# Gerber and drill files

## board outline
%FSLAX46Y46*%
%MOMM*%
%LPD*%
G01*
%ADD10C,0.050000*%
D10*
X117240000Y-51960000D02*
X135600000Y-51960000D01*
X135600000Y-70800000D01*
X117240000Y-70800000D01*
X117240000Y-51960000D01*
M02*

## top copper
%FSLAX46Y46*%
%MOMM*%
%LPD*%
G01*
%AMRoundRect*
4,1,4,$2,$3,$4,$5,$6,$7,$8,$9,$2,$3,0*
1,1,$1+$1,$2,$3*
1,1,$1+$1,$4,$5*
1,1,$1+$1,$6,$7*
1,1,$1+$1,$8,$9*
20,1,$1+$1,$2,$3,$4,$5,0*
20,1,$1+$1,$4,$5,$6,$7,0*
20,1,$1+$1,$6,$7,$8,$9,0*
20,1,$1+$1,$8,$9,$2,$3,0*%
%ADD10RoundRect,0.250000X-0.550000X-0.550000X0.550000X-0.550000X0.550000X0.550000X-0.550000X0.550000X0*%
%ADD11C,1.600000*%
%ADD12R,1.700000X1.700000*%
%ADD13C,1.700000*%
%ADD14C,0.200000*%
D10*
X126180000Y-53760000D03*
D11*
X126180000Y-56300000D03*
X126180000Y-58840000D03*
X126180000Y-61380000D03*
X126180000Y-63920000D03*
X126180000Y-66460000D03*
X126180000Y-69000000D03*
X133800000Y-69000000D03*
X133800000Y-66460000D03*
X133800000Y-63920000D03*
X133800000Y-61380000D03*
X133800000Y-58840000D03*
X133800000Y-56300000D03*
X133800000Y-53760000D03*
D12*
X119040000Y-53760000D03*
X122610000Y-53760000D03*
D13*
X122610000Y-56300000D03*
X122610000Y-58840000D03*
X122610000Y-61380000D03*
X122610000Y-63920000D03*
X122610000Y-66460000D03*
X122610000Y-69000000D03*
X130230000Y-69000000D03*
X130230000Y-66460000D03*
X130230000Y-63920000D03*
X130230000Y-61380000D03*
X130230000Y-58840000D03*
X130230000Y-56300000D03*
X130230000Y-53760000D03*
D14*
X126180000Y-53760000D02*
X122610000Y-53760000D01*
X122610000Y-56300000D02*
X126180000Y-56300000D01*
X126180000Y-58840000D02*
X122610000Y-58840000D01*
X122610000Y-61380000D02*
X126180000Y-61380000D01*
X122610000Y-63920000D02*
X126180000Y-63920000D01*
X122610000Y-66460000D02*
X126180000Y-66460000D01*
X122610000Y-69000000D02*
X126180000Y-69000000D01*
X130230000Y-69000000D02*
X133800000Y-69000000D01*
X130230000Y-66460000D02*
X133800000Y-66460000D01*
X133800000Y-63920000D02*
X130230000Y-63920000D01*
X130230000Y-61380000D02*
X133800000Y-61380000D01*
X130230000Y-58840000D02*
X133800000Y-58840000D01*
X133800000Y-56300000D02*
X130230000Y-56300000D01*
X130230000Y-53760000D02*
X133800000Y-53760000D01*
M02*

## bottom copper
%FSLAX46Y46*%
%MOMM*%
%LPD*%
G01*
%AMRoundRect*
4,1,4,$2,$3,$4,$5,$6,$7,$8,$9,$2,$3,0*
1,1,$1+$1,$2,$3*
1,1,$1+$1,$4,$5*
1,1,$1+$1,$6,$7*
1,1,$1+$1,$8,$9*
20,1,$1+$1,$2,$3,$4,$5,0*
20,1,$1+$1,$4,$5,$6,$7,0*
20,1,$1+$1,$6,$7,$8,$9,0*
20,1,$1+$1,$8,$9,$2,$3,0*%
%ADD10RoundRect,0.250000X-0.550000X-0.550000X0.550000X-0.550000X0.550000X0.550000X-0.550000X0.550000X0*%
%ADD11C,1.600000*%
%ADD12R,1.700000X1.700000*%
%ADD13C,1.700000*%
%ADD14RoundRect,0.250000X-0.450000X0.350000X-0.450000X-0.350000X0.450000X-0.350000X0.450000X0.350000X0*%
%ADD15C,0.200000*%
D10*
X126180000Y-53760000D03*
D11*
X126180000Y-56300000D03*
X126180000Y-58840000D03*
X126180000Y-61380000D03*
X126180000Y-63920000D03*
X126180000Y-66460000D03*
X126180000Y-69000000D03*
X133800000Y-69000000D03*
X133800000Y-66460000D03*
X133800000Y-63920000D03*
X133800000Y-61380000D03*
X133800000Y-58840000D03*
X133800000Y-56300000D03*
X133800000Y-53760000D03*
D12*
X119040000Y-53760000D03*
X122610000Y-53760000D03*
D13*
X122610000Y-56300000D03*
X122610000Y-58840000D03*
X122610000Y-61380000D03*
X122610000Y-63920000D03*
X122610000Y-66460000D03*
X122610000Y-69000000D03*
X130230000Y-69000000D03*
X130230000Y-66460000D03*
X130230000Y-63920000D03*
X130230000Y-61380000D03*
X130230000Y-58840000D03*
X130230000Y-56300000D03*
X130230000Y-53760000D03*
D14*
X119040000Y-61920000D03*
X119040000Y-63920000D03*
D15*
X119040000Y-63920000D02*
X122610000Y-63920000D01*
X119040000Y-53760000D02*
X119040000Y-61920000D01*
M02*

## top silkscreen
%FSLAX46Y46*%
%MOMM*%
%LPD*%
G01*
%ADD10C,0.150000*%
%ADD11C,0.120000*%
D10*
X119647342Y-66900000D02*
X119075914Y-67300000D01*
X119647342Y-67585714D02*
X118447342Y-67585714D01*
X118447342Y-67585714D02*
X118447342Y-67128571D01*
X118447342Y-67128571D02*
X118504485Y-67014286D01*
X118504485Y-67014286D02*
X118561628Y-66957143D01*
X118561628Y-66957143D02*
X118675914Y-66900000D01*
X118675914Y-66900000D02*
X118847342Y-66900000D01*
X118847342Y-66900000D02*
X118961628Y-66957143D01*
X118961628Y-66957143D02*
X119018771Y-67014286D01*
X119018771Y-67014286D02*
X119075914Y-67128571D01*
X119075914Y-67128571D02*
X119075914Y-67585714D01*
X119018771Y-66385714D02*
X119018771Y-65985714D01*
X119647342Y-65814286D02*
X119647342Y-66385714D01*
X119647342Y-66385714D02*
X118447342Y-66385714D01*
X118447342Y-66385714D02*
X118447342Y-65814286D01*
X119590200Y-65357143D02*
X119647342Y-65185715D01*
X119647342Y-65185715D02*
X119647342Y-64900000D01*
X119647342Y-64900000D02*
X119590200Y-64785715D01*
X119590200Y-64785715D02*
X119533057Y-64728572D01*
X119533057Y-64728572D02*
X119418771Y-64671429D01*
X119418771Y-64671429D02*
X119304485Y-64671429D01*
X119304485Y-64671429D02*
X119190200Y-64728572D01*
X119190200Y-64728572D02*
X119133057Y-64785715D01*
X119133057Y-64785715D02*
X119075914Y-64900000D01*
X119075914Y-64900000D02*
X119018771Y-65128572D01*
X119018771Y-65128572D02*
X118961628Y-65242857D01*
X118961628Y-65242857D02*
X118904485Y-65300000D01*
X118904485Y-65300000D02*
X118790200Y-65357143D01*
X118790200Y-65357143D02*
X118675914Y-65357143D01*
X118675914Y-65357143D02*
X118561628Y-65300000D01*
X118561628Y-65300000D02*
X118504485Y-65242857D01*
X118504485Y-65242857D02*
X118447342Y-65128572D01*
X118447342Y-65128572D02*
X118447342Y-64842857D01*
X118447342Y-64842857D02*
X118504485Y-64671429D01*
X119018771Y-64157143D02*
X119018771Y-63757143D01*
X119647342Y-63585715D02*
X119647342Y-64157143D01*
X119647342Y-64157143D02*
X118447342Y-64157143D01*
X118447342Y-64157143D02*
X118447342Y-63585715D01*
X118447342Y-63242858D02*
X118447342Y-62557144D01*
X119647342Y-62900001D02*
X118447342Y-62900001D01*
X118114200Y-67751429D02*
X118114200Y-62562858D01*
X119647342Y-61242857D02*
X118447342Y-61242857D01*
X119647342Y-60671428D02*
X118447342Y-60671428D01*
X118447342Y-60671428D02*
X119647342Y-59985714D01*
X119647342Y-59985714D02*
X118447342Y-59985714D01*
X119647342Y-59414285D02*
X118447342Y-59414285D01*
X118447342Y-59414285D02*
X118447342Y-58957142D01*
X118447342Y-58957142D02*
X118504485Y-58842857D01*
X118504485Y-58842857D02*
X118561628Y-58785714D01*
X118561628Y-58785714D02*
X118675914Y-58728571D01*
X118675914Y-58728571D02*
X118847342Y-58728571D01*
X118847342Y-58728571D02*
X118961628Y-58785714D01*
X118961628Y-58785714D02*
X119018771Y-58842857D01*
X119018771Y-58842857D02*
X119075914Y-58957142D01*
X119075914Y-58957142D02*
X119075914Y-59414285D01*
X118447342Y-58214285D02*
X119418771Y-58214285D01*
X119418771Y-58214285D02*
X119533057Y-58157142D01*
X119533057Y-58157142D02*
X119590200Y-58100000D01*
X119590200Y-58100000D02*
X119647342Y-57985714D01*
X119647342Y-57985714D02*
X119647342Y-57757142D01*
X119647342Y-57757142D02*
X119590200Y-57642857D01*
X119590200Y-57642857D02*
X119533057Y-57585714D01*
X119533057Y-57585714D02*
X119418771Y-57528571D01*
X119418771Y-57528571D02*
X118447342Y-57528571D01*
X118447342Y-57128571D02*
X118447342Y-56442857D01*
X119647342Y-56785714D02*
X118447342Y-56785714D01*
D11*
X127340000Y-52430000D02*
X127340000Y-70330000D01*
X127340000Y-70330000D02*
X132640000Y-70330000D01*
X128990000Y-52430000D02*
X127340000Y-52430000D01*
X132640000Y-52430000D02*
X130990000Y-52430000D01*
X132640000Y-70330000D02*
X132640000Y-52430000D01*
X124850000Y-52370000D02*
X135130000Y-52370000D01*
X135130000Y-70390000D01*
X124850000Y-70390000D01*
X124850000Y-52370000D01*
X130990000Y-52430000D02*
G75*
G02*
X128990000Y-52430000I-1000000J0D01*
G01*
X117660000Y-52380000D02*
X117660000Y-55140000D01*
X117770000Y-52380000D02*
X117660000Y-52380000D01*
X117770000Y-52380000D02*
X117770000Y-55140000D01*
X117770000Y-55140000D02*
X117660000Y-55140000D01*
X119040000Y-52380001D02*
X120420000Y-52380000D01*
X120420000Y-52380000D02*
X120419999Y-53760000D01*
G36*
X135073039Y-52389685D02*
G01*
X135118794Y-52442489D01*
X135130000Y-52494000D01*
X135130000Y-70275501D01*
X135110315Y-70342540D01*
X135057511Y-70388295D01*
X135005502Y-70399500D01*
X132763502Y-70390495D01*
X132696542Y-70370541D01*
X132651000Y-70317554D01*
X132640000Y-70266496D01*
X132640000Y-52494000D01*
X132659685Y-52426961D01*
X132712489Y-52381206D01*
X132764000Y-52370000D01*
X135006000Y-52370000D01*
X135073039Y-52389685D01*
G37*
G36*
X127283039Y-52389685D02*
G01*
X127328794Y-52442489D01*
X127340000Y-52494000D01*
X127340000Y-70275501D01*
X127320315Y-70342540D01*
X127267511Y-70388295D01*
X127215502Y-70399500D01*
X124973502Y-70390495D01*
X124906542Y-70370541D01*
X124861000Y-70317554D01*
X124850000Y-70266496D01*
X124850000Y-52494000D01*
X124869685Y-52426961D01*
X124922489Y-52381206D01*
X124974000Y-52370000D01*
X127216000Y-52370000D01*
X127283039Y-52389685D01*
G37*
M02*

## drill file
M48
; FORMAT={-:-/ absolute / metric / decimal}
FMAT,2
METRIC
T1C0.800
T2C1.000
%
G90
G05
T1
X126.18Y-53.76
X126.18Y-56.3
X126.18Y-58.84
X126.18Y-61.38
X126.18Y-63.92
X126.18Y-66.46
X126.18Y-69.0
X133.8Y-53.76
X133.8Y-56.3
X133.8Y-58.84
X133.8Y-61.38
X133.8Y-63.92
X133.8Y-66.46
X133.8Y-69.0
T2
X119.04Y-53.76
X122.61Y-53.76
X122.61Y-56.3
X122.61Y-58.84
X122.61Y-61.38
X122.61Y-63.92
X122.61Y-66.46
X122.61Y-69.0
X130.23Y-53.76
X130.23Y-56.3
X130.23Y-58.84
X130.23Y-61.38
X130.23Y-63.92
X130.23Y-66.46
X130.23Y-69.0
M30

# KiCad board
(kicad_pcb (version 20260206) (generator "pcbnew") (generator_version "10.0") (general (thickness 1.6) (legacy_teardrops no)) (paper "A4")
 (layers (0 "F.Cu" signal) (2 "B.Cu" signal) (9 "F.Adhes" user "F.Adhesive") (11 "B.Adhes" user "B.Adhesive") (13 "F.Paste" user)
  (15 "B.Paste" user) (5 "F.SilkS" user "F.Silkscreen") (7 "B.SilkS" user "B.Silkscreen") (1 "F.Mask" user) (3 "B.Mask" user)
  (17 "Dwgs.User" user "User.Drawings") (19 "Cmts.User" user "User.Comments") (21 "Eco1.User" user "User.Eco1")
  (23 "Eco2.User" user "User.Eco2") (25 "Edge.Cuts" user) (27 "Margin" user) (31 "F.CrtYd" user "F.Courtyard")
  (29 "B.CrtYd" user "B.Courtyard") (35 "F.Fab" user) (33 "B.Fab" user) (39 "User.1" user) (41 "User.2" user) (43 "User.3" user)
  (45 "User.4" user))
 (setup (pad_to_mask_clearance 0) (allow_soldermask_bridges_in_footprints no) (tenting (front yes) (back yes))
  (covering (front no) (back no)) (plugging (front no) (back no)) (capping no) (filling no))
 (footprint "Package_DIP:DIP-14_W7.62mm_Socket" (layer "F.Cu") (at 126.18 53.76)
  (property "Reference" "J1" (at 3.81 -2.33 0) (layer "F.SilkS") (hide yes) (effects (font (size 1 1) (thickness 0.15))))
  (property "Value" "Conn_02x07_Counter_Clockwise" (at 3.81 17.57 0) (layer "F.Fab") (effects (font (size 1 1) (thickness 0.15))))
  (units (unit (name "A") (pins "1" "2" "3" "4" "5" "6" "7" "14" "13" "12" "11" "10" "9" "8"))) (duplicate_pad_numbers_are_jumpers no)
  (fp_line (start 1.16 -1.33) (end 1.16 16.57) (stroke (width 0.12) (type solid)) (layer "F.SilkS"))
  (fp_line (start 1.16 16.57) (end 6.46 16.57) (stroke (width 0.12) (type solid)) (layer "F.SilkS"))
  (fp_line (start 2.81 -1.33) (end 1.16 -1.33) (stroke (width 0.12) (type solid)) (layer "F.SilkS"))
  (fp_line (start 6.46 -1.33) (end 4.81 -1.33) (stroke (width 0.12) (type solid)) (layer "F.SilkS"))
  (fp_line (start 6.46 16.57) (end 6.46 -1.33) (stroke (width 0.12) (type solid)) (layer "F.SilkS"))
  (fp_rect (start -1.33 -1.39) (end 8.95 16.63) (stroke (width 0.12) (type solid)) (fill no) (layer "F.SilkS"))
  (fp_arc (start 4.81 -1.33) (mid 3.81 -0.33) (end 2.81 -1.33) (stroke (width 0.12) (type solid)) (layer "F.SilkS"))
  (pad "1" thru_hole roundrect (at 0 0) (size 1.6 1.6) (drill 0.8) (layers "*.Cu" "*.Mask") (remove_unused_layers no)
   (roundrect_rratio 0.15625) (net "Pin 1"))
  (pad "2" thru_hole circle (at 0 2.54) (size 1.6 1.6) (drill 0.8) (layers "*.Cu" "*.Mask") (remove_unused_layers no) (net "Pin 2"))
  (pad "3" thru_hole circle (at 0 5.08) (size 1.6 1.6) (drill 0.8) (layers "*.Cu" "*.Mask") (remove_unused_layers no) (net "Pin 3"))
  (pad "4" thru_hole circle (at 0 7.62) (size 1.6 1.6) (drill 0.8) (layers "*.Cu" "*.Mask") (remove_unused_layers no) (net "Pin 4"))
  (pad "5" thru_hole circle (at 0 10.16) (size 1.6 1.6) (drill 0.8) (layers "*.Cu" "*.Mask") (remove_unused_layers no) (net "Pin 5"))
  (pad "6" thru_hole circle (at 0 12.7) (size 1.6 1.6) (drill 0.8) (layers "*.Cu" "*.Mask") (remove_unused_layers no) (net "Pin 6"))
  (pad "7" thru_hole circle (at 0 15.24) (size 1.6 1.6) (drill 0.8) (layers "*.Cu" "*.Mask") (remove_unused_layers no) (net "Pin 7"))
  (pad "8" thru_hole circle (at 7.62 15.24) (size 1.6 1.6) (drill 0.8) (layers "*.Cu" "*.Mask") (remove_unused_layers no) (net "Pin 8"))
  (pad "9" thru_hole circle (at 7.62 12.7) (size 1.6 1.6) (drill 0.8) (layers "*.Cu" "*.Mask") (remove_unused_layers no) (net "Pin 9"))
  (pad "10" thru_hole circle (at 7.62 10.16) (size 1.6 1.6) (drill 0.8) (layers "*.Cu" "*.Mask") (remove_unused_layers no) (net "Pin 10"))
  (pad "11" thru_hole circle (at 7.62 7.62) (size 1.6 1.6) (drill 0.8) (layers "*.Cu" "*.Mask") (remove_unused_layers no) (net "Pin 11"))
  (pad "12" thru_hole circle (at 7.62 5.08) (size 1.6 1.6) (drill 0.8) (layers "*.Cu" "*.Mask") (remove_unused_layers no) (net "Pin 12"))
  (pad "13" thru_hole circle (at 7.62 2.54) (size 1.6 1.6) (drill 0.8) (layers "*.Cu" "*.Mask") (remove_unused_layers no) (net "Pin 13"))
  (pad "14" thru_hole circle (at 7.62 0) (size 1.6 1.6) (drill 0.8) (layers "*.Cu" "*.Mask") (remove_unused_layers no) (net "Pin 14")))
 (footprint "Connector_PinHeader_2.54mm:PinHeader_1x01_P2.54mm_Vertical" (layer "F.Cu") (at 119.04 53.76 -90)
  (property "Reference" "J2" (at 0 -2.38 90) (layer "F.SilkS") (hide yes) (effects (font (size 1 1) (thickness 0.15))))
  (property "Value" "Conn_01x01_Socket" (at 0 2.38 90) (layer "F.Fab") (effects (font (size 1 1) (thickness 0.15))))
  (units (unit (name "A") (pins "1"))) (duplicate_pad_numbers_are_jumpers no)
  (fp_line (start -1.38 1.38) (end 1.38 1.38) (stroke (width 0.12) (type solid)) (layer "F.SilkS"))
  (fp_line (start -1.38 1.27) (end -1.38 1.38) (stroke (width 0.12) (type solid)) (layer "F.SilkS"))
  (fp_line (start -1.38 1.27) (end 1.38 1.27) (stroke (width 0.12) (type solid)) (layer "F.SilkS"))
  (fp_line (start 1.38 1.27) (end 1.38 1.38) (stroke (width 0.12) (type solid)) (layer "F.SilkS"))
  (fp_line (start -1.379999 0) (end -1.38 -1.38) (stroke (width 0.12) (type solid)) (layer "F.SilkS"))
  (fp_line (start -1.38 -1.38) (end 0 -1.379999) (stroke (width 0.12) (type solid)) (layer "F.SilkS"))
  (pad "1" thru_hole rect (at 0 0 270) (size 1.7 1.7) (drill 1) (layers "*.Cu" "*.Mask") (remove_unused_layers no) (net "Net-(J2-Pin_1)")))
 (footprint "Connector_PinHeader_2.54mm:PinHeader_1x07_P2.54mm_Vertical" (layer "B.Cu") (at 122.61 53.76 180)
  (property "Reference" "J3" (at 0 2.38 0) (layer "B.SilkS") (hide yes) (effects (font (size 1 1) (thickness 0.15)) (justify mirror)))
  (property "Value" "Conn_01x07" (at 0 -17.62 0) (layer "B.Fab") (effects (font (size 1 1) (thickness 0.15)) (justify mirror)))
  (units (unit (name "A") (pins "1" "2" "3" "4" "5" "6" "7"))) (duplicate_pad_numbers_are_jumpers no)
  (pad "1" thru_hole rect (at 0 0 180) (size 1.7 1.7) (drill 1) (layers "*.Cu" "*.Mask") (remove_unused_layers no) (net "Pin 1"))
  (pad "2" thru_hole circle (at 0 -2.54 180) (size 1.7 1.7) (drill 1) (layers "*.Cu" "*.Mask") (remove_unused_layers no) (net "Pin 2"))
  (pad "3" thru_hole circle (at 0 -5.08 180) (size 1.7 1.7) (drill 1) (layers "*.Cu" "*.Mask") (remove_unused_layers no) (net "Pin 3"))
  (pad "4" thru_hole circle (at 0 -7.62 180) (size 1.7 1.7) (drill 1) (layers "*.Cu" "*.Mask") (remove_unused_layers no) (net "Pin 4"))
  (pad "5" thru_hole circle (at 0 -10.16 180) (size 1.7 1.7) (drill 1) (layers "*.Cu" "*.Mask") (remove_unused_layers no) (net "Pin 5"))
  (pad "6" thru_hole circle (at 0 -12.7 180) (size 1.7 1.7) (drill 1) (layers "*.Cu" "*.Mask") (remove_unused_layers no) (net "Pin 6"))
  (pad "7" thru_hole circle (at 0 -15.24 180) (size 1.7 1.7) (drill 1) (layers "*.Cu" "*.Mask") (remove_unused_layers no) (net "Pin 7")))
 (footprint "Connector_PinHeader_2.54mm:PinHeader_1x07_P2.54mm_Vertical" (layer "B.Cu") (at 130.23 69)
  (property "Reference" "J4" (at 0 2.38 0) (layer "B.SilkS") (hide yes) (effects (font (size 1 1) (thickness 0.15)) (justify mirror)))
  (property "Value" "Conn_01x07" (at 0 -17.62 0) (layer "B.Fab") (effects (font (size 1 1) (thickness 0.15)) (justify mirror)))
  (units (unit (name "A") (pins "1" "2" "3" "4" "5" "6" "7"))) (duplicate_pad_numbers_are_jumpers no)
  (pad "1" thru_hole circle (at 0 0) (size 1.7 1.7) (drill 1) (layers "*.Cu" "*.Mask") (remove_unused_layers no) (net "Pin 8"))
  (pad "2" thru_hole circle (at 0 -2.54) (size 1.7 1.7) (drill 1) (layers "*.Cu" "*.Mask") (remove_unused_layers no) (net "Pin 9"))
  (pad "3" thru_hole circle (at 0 -5.08) (size 1.7 1.7) (drill 1) (layers "*.Cu" "*.Mask") (remove_unused_layers no) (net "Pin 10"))
  (pad "4" thru_hole circle (at 0 -7.62) (size 1.7 1.7) (drill 1) (layers "*.Cu" "*.Mask") (remove_unused_layers no) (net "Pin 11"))
  (pad "5" thru_hole circle (at 0 -10.16) (size 1.7 1.7) (drill 1) (layers "*.Cu" "*.Mask") (remove_unused_layers no) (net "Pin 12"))
  (pad "6" thru_hole circle (at 0 -12.7) (size 1.7 1.7) (drill 1) (layers "*.Cu" "*.Mask") (remove_unused_layers no) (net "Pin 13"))
  (pad "7" thru_hole circle (at 0 -15.24) (size 1.7 1.7) (drill 1) (layers "*.Cu" "*.Mask") (remove_unused_layers no) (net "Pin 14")))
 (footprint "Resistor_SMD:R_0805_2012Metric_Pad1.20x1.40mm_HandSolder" (layer "B.Cu") (at 119.04 62.92 -90)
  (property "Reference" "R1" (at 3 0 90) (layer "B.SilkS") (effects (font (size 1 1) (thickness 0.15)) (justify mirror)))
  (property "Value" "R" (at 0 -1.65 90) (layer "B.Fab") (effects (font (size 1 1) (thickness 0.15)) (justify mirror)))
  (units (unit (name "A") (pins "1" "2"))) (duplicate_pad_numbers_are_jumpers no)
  (pad "1" smd roundrect (at -1 0 270) (size 1.2 1.4) (layers "B.Cu" "B.Mask" "B.Paste") (roundrect_rratio 0.208333) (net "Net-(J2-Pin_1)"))
  (pad "2" smd roundrect (at 1 0 270) (size 1.2 1.4) (layers "B.Cu" "B.Mask" "B.Paste") (roundrect_rratio 0.208333) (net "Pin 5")))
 (gr_rect (start 117.24 51.96) (end 135.6 70.8) (stroke (width 0.05) (type solid)) (fill no) (layer "Edge.Cuts"))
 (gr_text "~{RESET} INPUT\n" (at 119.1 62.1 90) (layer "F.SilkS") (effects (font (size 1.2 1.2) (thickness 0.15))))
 (segment (start 126.18 53.76) (end 122.61 53.76) (width 0.2) (layer "F.Cu") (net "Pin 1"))
 (segment (start 122.61 56.3) (end 126.18 56.3) (width 0.2) (layer "F.Cu") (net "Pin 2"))
 (segment (start 126.18 58.84) (end 122.61 58.84) (width 0.2) (layer "F.Cu") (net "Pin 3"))
 (segment (start 122.61 61.38) (end 126.18 61.38) (width 0.2) (layer "F.Cu") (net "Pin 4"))
 (segment (start 122.61 63.92) (end 126.18 63.92) (width 0.2) (layer "F.Cu") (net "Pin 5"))
 (segment (start 119.04 63.92) (end 122.61 63.92) (width 0.2) (layer "B.Cu") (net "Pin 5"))
 (segment (start 122.61 66.46) (end 126.18 66.46) (width 0.2) (layer "F.Cu") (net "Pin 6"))
 (segment (start 122.61 69) (end 126.18 69) (width 0.2) (layer "F.Cu") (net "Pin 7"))
 (segment (start 130.23 69) (end 133.8 69) (width 0.2) (layer "F.Cu") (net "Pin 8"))
 (segment (start 130.23 66.46) (end 133.8 66.46) (width 0.2) (layer "F.Cu") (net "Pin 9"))
 (segment (start 133.8 63.92) (end 130.23 63.92) (width 0.2) (layer "F.Cu") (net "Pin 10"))
 (segment (start 130.23 61.38) (end 133.8 61.38) (width 0.2) (layer "F.Cu") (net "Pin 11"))
 (segment (start 130.23 58.84) (end 133.8 58.84) (width 0.2) (layer "F.Cu") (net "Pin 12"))
 (segment (start 133.8 56.3) (end 130.23 56.3) (width 0.2) (layer "F.Cu") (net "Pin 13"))
 (segment (start 130.23 53.76) (end 133.8 53.76) (width 0.2) (layer "F.Cu") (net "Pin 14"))
 (segment (start 119.04 53.76) (end 119.04 61.92) (width 0.2) (layer "B.Cu") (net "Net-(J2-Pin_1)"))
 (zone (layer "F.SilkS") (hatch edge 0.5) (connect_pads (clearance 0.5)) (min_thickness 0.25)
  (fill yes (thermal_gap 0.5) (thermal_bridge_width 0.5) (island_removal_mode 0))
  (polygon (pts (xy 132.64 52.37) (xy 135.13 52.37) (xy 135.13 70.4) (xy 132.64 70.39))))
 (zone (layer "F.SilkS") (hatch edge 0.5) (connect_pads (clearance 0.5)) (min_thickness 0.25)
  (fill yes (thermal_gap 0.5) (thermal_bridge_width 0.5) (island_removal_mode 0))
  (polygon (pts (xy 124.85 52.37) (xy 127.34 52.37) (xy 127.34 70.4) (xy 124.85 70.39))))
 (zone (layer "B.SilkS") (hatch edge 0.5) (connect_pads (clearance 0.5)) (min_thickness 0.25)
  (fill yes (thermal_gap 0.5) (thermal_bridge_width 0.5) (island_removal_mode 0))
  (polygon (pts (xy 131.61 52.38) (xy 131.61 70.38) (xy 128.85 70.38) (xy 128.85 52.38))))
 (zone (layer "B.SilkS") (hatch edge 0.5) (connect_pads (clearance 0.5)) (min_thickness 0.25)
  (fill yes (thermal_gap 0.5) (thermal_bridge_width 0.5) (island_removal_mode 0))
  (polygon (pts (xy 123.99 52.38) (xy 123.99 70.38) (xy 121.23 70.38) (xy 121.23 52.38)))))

